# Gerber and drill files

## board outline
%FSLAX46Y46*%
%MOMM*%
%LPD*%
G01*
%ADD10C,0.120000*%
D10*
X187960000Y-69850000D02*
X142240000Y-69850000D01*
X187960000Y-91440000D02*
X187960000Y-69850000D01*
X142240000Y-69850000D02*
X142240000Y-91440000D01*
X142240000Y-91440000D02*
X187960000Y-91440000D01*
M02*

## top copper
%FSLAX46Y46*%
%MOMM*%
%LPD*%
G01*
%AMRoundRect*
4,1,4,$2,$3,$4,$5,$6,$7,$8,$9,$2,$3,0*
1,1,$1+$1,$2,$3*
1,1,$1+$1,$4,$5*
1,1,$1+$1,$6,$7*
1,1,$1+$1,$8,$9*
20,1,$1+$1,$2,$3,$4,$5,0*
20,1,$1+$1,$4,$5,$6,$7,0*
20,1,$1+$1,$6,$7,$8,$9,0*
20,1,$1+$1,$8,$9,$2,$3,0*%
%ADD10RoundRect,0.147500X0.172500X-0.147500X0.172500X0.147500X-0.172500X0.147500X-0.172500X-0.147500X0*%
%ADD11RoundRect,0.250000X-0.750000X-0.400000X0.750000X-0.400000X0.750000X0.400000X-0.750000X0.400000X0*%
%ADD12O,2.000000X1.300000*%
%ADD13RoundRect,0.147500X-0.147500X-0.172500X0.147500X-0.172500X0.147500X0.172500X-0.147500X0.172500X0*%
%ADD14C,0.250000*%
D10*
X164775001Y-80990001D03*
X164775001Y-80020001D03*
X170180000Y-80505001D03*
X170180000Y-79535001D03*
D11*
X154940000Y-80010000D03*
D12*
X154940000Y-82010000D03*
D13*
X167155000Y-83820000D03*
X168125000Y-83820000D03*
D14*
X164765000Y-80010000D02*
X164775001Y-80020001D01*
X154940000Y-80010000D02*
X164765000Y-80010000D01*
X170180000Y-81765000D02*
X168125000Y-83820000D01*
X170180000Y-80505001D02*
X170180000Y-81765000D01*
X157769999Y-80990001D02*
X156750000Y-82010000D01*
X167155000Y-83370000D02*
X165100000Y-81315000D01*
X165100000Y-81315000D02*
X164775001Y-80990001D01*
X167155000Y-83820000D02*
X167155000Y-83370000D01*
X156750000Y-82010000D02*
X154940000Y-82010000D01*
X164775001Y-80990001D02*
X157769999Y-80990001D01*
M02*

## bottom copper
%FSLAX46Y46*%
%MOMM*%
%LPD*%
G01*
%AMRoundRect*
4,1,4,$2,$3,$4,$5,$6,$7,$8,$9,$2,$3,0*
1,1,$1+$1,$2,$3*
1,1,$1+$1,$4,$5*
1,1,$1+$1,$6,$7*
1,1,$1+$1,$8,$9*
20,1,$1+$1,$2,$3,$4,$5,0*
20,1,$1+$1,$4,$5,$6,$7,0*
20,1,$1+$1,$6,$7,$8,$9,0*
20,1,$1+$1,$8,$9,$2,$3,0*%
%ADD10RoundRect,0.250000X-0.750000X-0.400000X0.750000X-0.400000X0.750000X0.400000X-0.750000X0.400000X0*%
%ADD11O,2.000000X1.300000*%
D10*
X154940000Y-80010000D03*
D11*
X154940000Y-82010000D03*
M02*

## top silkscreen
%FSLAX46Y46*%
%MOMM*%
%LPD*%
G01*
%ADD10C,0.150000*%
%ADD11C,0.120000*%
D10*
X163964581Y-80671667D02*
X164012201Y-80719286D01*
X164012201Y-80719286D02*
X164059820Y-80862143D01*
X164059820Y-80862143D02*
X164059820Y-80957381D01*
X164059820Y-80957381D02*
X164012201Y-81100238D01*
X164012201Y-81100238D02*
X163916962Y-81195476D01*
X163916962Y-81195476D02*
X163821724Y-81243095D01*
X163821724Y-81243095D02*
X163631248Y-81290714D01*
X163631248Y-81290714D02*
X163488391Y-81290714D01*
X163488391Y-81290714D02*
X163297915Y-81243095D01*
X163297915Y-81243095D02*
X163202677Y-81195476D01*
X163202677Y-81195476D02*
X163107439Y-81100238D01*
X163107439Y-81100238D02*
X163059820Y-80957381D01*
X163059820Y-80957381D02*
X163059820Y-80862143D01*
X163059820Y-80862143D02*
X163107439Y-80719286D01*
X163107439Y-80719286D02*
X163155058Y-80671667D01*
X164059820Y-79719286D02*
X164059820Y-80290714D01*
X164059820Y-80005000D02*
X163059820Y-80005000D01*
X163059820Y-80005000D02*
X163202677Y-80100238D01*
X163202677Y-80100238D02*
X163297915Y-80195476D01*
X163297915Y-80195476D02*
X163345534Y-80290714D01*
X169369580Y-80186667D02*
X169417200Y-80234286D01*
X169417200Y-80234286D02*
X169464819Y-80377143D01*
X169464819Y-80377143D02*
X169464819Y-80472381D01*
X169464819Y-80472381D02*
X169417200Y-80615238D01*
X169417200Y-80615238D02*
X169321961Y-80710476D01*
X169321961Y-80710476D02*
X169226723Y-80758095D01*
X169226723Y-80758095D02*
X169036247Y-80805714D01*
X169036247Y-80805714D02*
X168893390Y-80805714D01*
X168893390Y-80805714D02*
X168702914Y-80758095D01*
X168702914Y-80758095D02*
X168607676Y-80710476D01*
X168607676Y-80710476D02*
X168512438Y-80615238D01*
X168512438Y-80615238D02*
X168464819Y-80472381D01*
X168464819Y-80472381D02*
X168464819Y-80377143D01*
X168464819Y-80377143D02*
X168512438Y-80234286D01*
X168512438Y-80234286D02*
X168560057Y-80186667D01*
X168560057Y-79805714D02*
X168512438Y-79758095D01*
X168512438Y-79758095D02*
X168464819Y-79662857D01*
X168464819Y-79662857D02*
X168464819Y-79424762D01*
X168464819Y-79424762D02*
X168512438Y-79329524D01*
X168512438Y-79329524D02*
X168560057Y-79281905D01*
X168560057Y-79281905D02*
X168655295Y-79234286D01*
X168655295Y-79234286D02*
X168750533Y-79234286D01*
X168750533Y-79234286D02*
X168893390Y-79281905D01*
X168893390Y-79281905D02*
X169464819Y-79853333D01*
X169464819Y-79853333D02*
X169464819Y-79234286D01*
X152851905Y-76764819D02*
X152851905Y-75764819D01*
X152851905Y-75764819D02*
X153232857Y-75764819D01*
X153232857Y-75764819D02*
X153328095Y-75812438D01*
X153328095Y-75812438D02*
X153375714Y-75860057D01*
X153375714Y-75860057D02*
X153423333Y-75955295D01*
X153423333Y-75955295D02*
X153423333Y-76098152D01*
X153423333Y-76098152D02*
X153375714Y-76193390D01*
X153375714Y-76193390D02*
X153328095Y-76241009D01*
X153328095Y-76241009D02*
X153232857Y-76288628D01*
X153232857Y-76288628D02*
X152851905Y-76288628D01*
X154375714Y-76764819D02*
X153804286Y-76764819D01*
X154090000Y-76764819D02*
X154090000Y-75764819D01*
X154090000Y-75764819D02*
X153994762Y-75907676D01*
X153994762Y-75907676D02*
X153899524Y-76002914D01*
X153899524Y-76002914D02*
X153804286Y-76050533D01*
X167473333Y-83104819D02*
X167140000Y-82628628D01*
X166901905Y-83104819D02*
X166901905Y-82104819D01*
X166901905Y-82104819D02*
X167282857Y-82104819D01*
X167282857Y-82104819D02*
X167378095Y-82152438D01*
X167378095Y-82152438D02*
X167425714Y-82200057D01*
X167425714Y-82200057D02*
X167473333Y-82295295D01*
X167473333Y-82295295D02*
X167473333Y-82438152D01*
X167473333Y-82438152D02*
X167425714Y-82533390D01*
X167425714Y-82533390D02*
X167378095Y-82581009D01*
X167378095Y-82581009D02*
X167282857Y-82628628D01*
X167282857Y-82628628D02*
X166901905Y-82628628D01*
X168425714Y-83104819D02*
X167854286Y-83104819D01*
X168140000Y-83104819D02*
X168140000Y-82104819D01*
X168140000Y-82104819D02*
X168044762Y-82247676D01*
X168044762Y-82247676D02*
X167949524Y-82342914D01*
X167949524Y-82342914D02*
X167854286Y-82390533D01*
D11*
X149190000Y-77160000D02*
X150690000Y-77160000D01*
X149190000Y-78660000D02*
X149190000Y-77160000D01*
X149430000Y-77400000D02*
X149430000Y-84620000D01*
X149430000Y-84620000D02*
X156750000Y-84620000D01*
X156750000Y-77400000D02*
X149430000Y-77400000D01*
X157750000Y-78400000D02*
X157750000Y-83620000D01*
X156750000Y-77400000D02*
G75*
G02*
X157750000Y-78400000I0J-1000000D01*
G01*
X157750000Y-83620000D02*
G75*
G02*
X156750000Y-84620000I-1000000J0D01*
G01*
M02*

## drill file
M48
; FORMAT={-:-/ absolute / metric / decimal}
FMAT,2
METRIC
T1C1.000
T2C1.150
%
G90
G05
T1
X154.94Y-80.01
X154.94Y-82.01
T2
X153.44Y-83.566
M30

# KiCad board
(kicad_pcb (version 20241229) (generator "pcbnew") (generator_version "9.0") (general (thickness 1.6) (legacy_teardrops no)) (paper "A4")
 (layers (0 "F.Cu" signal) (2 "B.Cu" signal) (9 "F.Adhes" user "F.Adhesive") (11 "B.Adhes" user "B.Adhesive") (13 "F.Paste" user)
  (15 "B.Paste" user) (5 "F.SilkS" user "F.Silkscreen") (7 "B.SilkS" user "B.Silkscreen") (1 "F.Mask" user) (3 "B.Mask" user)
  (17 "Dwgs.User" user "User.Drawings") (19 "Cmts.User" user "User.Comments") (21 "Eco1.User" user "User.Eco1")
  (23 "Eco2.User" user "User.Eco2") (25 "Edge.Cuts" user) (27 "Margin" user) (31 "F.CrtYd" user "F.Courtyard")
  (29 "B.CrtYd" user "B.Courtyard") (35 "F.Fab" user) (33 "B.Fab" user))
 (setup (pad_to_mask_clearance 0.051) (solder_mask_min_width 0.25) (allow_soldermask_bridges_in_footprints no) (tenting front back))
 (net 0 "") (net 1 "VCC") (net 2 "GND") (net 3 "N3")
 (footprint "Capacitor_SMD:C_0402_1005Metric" (layer "F.Cu") (at 164.775001 80.505001 90)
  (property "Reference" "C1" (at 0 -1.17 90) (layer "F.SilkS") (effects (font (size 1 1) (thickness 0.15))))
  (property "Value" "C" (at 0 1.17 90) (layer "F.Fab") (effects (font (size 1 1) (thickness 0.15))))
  (pad "1" smd roundrect (at -0.485 0 90) (size 0.59 0.64) (layers "F.Cu" "F.Mask" "F.Paste") (roundrect_rratio 0.25) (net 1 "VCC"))
  (pad "2" smd roundrect (at 0.485 0 90) (size 0.59 0.64) (layers "F.Cu" "F.Mask" "F.Paste") (roundrect_rratio 0.25) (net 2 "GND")))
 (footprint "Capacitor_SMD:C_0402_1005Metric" (layer "F.Cu") (at 170.18 80.020001 90)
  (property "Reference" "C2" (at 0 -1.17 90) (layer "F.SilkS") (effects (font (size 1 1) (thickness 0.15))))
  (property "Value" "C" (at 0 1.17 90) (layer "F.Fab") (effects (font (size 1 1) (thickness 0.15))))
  (pad "1" smd roundrect (at -0.485 0 90) (size 0.59 0.64) (layers "F.Cu" "F.Mask" "F.Paste") (roundrect_rratio 0.25) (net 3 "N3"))
  (pad "2" smd roundrect (at 0.485 0 90) (size 0.59 0.64) (layers "F.Cu" "F.Mask" "F.Paste") (roundrect_rratio 0.25) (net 2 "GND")))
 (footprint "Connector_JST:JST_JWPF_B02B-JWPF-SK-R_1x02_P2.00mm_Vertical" (layer "F.Cu") (at 154.94 80.01)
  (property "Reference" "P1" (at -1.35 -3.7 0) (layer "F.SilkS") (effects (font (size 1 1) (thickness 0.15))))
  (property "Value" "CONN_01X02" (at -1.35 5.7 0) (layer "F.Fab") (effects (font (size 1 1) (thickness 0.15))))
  (fp_line (start -5.75 -2.85) (end -4.25 -2.85) (stroke (width 0.12) (type solid)) (layer "F.SilkS"))
  (fp_line (start -5.75 -1.35) (end -5.75 -2.85) (stroke (width 0.12) (type solid)) (layer "F.SilkS"))
  (fp_line (start -5.51 -2.61) (end -5.51 4.61) (stroke (width 0.12) (type solid)) (layer "F.SilkS"))
  (fp_line (start -5.51 4.61) (end 1.81 4.61) (stroke (width 0.12) (type solid)) (layer "F.SilkS"))
  (fp_line (start 1.81 -2.61) (end -5.51 -2.61) (stroke (width 0.12) (type solid)) (layer "F.SilkS"))
  (fp_line (start 2.81 -1.61) (end 2.81 3.61) (stroke (width 0.12) (type solid)) (layer "F.SilkS"))
  (fp_arc (start 1.81 -2.61) (mid 2.517107 -2.317107) (end 2.81 -1.61) (stroke (width 0.12) (type solid)) (layer "F.SilkS"))
  (fp_arc (start 2.81 3.61) (mid 2.517107 4.317107) (end 1.81 4.61) (stroke (width 0.12) (type solid)) (layer "F.SilkS"))
  (pad "" np_thru_hole circle (at -1.5 3.556) (size 1.15 1.15) (drill 1.15) (layers "*.Cu" "*.Mask"))
  (pad "1" thru_hole roundrect (at 0 0) (size 2 1.3) (drill 1) (layers "*.Cu" "*.Mask") (remove_unused_layers no)
   (roundrect_rratio 0.192308) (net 2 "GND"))
  (pad "2" thru_hole oval (at 0 2) (size 2 1.3) (drill 1) (layers "*.Cu" "*.Mask") (remove_unused_layers no) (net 1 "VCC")))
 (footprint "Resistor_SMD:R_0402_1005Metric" (layer "F.Cu") (at 167.64 83.82)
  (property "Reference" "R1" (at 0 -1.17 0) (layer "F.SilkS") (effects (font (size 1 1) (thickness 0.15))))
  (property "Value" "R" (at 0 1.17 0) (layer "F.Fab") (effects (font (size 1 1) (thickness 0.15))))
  (pad "1" smd roundrect (at -0.485 0) (size 0.59 0.64) (layers "F.Cu" "F.Mask" "F.Paste") (roundrect_rratio 0.25) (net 1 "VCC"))
  (pad "2" smd roundrect (at 0.485 0) (size 0.59 0.64) (layers "F.Cu" "F.Mask" "F.Paste") (roundrect_rratio 0.25) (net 3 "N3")))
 (gr_line (start 187.96 69.85) (end 142.24 69.85) (stroke (width 0.12) (type solid)) (layer "Edge.Cuts"))
 (gr_line (start 187.96 91.44) (end 187.96 69.85) (stroke (width 0.12) (type solid)) (layer "Edge.Cuts"))
 (gr_line (start 142.24 69.85) (end 142.24 91.44) (stroke (width 0.12) (type solid)) (layer "Edge.Cuts"))
 (gr_line (start 142.24 91.44) (end 187.96 91.44) (stroke (width 0.12) (type solid)) (layer "Edge.Cuts"))
 (segment (start 164.765 80.01) (end 164.775001 80.020001) (width 0.25) (layer "F.Cu") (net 2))
 (segment (start 154.94 80.01) (end 164.765 80.01) (width 0.25) (layer "F.Cu") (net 2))
 (segment (start 170.18 81.765) (end 168.125 83.82) (width 0.25) (layer "F.Cu") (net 3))
 (segment (start 170.18 80.505001) (end 170.18 81.765) (width 0.25) (layer "F.Cu") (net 3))
 (segment (start 157.769999 80.990001) (end 156.75 82.01) (width 0.25) (layer "F.Cu") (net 1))
 (segment (start 167.155 83.37) (end 165.1 81.315) (width 0.25) (layer "F.Cu") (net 1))
 (segment (start 165.1 81.315) (end 164.775001 80.990001) (width 0.25) (layer "F.Cu") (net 1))
 (segment (start 167.155 83.82) (end 167.155 83.37) (width 0.25) (layer "F.Cu") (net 1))
 (segment (start 156.75 82.01) (end 154.94 82.01) (width 0.25) (layer "F.Cu") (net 1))
 (segment (start 164.775001 80.990001) (end 157.769999 80.990001) (width 0.25) (layer "F.Cu") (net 1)))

